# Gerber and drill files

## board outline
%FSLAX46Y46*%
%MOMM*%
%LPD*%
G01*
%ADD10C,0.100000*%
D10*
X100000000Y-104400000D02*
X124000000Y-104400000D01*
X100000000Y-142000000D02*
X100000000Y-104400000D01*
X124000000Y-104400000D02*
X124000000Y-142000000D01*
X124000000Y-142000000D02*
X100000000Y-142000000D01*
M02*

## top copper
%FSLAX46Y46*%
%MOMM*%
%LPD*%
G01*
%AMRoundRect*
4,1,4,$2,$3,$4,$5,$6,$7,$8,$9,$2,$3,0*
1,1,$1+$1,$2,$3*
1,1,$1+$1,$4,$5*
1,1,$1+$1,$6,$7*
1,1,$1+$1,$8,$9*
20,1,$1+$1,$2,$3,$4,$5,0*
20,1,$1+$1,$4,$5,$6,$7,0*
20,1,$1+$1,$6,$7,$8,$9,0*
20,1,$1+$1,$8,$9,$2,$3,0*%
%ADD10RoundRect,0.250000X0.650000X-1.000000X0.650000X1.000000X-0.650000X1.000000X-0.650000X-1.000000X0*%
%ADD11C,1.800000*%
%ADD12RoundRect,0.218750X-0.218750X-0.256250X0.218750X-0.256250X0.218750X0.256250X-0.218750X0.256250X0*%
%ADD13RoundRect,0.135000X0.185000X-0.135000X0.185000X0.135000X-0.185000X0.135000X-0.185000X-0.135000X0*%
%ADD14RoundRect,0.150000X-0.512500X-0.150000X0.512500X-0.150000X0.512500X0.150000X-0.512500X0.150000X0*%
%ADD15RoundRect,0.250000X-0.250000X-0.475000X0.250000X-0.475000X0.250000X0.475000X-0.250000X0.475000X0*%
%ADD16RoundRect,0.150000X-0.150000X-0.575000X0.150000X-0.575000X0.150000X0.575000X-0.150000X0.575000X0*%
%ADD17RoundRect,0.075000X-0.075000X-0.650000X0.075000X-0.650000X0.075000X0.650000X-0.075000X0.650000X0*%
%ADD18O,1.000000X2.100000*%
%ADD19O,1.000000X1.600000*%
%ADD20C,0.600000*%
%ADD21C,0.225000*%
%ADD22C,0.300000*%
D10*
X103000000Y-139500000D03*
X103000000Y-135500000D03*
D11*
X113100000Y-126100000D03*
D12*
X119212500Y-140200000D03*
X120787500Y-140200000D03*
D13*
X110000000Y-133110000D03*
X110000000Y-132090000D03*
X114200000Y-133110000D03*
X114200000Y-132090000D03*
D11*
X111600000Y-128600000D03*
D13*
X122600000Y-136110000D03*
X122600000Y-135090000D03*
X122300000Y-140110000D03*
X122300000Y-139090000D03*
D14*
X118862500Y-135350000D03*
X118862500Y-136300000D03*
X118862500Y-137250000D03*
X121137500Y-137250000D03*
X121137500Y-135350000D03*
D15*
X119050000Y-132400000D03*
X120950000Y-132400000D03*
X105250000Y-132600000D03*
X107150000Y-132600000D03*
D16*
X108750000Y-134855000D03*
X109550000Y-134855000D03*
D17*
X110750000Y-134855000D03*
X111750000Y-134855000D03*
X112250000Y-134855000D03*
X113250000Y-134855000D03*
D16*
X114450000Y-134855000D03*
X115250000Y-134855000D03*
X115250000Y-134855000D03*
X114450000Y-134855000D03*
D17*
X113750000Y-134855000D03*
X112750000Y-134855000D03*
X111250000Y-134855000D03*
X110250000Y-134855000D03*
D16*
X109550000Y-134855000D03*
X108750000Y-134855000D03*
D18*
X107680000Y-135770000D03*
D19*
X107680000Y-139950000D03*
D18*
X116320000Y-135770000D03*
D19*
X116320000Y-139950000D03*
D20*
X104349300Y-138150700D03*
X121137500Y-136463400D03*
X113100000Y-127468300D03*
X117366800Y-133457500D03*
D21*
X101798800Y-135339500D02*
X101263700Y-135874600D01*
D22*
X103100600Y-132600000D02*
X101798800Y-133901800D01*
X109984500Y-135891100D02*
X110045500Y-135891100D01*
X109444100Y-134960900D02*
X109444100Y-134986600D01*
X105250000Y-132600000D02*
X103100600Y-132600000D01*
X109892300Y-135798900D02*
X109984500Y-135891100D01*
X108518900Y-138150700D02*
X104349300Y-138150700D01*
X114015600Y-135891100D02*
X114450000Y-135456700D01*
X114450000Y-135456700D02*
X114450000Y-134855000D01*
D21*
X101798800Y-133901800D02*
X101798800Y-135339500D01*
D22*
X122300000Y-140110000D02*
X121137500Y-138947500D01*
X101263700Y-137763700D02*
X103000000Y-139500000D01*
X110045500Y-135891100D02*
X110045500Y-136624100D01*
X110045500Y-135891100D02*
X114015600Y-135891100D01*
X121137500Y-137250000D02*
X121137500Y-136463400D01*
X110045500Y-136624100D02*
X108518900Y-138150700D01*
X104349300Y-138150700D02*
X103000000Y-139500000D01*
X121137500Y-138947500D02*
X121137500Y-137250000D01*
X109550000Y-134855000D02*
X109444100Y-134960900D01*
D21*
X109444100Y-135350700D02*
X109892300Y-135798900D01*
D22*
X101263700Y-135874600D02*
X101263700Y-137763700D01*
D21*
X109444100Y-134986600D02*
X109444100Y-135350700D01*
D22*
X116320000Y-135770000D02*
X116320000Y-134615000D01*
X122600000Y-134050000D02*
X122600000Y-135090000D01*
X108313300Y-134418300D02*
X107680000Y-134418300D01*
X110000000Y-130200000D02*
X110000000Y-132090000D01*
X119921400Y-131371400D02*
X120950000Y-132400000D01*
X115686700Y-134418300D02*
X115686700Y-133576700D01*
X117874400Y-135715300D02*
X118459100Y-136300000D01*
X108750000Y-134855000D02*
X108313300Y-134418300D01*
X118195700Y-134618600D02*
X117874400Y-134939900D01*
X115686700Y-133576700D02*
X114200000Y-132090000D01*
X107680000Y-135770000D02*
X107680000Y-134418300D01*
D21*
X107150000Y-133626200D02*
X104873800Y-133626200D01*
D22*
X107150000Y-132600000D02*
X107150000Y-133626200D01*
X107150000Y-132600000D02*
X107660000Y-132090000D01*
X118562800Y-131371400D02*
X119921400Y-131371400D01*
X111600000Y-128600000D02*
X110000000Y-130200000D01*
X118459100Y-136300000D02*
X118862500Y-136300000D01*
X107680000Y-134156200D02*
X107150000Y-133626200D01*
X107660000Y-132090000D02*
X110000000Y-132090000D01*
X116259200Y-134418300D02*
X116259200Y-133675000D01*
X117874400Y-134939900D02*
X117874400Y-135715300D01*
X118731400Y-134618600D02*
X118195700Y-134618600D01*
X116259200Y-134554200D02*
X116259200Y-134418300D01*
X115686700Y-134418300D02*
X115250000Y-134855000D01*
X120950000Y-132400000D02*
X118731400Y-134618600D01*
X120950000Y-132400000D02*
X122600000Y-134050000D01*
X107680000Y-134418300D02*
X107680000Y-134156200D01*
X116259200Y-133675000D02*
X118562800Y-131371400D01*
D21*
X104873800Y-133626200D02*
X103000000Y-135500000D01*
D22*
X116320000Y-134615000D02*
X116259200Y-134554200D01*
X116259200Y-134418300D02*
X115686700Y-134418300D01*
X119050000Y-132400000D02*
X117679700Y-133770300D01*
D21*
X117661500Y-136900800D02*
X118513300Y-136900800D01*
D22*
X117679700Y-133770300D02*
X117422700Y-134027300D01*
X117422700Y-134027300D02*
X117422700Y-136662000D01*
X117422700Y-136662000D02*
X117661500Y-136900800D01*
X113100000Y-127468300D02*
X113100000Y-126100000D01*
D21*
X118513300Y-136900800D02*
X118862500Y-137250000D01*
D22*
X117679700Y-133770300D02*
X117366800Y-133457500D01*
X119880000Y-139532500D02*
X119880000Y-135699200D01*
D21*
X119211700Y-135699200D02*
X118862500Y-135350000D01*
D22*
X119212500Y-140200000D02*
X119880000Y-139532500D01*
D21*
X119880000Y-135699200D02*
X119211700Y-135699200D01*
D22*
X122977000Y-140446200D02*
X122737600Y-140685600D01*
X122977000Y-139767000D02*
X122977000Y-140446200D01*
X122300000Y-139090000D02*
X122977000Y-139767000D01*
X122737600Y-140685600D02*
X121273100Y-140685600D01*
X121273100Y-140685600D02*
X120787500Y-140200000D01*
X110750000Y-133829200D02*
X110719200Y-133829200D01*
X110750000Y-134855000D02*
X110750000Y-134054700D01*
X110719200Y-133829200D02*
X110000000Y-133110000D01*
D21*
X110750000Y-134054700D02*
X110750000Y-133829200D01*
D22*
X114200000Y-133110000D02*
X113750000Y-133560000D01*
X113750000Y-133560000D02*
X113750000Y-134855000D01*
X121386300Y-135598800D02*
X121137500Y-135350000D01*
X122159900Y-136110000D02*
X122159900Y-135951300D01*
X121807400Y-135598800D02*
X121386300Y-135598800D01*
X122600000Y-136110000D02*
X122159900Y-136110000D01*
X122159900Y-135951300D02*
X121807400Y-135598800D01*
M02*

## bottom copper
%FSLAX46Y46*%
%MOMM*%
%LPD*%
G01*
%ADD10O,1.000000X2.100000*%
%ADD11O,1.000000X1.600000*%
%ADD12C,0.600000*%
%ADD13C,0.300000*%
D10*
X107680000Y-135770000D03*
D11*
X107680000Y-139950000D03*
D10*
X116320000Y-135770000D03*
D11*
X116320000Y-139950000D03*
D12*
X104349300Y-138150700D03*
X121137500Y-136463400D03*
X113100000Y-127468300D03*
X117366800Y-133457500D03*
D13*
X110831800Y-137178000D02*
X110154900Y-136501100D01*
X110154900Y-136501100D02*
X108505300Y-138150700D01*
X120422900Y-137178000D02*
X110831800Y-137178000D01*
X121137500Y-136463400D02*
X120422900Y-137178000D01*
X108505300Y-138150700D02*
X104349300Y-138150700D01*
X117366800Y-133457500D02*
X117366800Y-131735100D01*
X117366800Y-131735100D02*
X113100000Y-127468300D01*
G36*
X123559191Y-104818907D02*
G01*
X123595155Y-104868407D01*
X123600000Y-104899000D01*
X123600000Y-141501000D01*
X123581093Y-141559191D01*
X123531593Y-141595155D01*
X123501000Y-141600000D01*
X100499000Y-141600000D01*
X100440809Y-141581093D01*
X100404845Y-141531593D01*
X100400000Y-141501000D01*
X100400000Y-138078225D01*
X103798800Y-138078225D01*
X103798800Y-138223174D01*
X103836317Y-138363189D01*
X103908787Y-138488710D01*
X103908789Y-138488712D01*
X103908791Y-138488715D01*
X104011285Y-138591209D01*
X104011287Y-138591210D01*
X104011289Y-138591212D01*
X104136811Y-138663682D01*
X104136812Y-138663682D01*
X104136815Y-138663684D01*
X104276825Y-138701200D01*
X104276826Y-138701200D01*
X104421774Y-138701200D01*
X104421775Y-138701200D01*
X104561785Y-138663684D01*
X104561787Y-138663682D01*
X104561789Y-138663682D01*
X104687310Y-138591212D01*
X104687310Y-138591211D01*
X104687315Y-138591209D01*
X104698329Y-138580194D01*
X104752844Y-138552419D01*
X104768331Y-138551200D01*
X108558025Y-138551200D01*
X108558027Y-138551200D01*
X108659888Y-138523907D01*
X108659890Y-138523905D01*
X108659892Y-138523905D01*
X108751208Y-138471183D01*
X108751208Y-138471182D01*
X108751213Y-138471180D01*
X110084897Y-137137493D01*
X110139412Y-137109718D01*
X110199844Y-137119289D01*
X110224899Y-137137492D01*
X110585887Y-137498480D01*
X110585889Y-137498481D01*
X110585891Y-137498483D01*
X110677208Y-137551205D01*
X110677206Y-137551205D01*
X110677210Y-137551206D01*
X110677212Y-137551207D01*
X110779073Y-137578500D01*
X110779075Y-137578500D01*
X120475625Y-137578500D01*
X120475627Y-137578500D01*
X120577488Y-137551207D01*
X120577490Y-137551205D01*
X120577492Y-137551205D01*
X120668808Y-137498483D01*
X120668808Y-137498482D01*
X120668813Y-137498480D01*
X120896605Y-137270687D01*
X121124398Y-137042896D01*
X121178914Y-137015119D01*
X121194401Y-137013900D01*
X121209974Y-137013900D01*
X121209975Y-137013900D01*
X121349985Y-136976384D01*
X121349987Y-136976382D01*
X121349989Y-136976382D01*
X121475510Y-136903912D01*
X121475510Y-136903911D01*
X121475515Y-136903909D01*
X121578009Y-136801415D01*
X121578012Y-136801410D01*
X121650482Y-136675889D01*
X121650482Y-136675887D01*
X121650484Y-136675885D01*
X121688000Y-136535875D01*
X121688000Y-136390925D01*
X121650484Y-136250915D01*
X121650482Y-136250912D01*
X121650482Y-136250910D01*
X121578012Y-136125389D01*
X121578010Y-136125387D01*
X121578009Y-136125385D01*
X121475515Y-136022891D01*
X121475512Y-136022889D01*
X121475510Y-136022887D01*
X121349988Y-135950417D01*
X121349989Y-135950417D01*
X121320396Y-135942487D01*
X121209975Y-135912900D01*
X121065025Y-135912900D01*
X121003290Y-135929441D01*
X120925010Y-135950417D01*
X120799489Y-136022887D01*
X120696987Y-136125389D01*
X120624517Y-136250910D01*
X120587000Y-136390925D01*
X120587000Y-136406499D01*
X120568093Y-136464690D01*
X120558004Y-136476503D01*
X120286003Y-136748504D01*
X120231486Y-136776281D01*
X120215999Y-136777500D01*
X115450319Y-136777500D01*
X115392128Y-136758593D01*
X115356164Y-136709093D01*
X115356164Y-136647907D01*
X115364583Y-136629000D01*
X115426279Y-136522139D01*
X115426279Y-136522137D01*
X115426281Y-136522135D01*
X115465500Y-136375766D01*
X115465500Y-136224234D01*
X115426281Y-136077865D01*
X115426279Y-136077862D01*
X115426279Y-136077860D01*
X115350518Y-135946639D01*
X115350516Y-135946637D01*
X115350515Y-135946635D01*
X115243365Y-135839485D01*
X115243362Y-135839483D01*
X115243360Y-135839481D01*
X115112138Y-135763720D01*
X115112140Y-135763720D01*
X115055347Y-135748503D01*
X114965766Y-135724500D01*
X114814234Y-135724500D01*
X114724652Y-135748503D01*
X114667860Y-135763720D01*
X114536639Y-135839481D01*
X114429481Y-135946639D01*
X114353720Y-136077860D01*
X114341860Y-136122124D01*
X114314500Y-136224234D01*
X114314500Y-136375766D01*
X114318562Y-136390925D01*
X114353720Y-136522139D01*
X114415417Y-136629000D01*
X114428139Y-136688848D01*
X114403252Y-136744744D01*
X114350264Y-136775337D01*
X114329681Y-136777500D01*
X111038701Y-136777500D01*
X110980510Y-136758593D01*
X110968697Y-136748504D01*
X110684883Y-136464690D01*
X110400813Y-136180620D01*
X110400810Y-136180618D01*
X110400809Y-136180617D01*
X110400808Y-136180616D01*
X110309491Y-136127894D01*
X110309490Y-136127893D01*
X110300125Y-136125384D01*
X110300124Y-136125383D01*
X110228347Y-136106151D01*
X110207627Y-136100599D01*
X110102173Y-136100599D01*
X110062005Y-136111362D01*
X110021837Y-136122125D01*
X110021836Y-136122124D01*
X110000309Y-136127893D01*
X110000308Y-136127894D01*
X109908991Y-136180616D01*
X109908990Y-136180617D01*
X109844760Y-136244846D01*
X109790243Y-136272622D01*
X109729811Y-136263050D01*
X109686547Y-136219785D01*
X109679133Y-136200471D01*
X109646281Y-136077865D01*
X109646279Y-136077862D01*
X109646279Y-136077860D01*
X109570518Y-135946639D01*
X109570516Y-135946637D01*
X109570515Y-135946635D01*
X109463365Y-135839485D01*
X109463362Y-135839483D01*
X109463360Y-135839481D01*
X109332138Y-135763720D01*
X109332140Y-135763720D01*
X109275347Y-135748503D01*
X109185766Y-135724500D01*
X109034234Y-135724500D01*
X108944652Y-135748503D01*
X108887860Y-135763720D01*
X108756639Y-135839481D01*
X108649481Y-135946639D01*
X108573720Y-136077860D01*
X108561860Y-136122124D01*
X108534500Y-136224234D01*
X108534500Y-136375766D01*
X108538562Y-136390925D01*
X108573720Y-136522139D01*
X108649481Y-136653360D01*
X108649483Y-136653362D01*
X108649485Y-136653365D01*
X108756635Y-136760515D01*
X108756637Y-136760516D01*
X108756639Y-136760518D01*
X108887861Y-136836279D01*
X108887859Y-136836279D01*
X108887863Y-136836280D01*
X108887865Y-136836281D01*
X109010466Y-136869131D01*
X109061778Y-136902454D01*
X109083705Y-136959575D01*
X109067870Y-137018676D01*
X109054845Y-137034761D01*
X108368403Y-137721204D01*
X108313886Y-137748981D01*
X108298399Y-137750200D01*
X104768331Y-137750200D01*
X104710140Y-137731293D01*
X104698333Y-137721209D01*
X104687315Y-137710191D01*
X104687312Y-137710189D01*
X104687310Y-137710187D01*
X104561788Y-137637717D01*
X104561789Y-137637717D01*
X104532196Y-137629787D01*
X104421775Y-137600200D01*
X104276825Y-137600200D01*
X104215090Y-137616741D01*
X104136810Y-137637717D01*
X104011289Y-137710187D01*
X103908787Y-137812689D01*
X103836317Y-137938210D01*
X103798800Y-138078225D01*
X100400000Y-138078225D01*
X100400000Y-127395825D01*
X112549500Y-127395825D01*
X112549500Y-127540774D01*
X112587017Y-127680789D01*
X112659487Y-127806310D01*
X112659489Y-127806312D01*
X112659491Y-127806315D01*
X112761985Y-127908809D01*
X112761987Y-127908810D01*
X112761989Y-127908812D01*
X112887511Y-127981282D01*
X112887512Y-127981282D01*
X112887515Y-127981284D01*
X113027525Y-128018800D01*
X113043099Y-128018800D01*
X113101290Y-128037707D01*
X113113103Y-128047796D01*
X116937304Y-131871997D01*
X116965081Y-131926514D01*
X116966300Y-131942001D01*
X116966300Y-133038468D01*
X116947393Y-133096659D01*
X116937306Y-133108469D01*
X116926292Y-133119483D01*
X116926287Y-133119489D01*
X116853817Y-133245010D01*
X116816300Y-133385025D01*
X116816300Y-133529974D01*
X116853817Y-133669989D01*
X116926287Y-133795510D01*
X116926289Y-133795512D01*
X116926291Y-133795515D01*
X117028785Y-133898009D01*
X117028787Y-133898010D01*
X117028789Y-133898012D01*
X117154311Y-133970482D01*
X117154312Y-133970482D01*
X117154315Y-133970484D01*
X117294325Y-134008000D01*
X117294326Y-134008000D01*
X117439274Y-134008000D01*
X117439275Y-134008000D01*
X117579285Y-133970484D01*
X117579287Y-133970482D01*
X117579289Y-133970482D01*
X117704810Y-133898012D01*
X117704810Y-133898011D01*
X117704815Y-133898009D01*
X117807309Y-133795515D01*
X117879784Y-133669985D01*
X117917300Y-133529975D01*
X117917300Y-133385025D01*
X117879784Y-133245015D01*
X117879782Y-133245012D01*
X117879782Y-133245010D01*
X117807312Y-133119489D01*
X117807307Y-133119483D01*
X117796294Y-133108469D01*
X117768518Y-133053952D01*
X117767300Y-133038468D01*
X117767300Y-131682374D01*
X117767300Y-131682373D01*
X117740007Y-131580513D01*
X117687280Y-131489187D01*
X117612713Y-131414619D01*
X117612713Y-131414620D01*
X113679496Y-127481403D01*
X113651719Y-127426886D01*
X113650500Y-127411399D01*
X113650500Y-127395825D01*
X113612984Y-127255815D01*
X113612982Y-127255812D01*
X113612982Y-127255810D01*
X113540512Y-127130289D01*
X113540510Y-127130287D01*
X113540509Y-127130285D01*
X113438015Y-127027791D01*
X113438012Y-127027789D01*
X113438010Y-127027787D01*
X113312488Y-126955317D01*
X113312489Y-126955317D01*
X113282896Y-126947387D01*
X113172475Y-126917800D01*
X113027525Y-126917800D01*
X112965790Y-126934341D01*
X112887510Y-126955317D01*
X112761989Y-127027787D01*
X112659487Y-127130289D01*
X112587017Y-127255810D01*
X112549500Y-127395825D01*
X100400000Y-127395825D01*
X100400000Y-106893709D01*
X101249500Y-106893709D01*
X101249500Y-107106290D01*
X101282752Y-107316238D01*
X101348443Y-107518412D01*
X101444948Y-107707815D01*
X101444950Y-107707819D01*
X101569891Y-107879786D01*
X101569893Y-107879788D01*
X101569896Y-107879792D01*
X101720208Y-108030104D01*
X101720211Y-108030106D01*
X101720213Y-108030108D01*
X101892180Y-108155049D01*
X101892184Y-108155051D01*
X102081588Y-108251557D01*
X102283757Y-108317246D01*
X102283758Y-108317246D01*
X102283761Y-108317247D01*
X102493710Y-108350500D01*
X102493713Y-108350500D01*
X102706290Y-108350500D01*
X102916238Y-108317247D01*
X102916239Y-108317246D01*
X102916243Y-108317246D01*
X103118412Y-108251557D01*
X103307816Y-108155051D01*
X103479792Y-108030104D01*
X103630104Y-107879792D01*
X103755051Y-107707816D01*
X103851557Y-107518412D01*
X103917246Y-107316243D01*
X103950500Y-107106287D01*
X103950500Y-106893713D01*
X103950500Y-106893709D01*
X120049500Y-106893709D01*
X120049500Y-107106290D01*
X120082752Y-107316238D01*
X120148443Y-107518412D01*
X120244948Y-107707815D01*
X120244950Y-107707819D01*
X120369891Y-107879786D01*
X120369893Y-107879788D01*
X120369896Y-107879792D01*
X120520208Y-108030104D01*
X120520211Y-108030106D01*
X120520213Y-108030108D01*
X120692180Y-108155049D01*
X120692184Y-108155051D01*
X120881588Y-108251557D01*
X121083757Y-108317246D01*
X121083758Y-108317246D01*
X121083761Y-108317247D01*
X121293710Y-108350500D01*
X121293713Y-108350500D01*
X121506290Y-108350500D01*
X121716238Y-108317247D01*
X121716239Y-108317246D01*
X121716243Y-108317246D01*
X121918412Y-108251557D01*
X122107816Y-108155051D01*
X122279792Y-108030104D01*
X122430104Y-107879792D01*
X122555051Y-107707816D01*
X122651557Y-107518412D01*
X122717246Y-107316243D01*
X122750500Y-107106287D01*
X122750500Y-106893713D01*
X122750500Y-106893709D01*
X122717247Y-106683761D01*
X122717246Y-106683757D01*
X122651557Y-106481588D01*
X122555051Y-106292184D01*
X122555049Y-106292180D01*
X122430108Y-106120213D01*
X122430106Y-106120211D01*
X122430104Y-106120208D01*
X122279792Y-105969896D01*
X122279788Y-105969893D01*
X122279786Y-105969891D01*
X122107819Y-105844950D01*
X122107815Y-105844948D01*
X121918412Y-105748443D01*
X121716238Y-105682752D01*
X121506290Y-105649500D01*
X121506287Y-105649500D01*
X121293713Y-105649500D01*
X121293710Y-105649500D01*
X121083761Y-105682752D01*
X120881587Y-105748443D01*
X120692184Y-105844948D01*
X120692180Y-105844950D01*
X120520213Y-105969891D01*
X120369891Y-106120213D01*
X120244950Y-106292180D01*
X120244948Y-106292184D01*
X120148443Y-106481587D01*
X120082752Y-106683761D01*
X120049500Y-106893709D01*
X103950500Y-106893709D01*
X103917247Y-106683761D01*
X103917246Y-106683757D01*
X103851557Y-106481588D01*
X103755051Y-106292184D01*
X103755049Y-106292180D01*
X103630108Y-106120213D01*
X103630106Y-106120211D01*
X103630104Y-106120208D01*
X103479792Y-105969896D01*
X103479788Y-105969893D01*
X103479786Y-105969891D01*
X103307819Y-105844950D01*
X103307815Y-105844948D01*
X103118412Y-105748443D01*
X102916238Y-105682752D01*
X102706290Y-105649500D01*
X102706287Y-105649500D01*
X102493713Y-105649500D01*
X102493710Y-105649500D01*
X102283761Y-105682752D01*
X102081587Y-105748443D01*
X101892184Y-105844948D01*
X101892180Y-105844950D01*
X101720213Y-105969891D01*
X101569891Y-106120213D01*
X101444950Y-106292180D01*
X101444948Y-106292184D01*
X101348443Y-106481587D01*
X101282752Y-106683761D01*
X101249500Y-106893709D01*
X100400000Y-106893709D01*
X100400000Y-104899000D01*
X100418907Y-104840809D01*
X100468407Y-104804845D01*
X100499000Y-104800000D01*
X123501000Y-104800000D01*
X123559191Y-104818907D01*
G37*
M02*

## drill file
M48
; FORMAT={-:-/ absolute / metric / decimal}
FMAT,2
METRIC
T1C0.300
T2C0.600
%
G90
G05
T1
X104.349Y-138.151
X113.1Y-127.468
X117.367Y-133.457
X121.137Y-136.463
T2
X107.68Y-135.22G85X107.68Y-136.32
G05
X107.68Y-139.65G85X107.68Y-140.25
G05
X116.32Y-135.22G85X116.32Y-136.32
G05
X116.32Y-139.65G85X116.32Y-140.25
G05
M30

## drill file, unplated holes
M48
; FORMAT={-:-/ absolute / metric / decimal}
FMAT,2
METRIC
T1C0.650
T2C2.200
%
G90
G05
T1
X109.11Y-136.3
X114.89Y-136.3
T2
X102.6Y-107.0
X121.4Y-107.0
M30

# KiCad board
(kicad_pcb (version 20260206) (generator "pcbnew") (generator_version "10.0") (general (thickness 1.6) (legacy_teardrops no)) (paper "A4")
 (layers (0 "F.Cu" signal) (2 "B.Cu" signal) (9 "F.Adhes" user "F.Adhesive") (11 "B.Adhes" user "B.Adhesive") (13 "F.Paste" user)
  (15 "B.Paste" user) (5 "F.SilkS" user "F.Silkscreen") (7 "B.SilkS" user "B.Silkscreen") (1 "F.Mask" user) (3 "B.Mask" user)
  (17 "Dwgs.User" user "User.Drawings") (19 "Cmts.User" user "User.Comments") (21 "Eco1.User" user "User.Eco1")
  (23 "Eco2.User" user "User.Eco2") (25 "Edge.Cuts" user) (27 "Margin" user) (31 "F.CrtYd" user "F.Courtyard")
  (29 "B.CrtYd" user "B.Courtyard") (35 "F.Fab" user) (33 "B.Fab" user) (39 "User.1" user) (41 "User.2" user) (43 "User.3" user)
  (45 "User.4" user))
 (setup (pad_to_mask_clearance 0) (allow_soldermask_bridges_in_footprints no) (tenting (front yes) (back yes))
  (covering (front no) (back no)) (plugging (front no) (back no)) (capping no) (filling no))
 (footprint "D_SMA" (layer "F.Cu") (at 103 137.5 90)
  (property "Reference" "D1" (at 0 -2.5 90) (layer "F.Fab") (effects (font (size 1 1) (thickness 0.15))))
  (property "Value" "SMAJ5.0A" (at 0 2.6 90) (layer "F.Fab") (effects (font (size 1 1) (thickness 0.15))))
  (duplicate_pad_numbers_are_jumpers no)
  (pad "1" smd roundrect (at -2 0 90) (size 2.5 1.8) (layers "F.Cu" "F.Mask" "F.Paste") (roundrect_rratio 0.1388888889) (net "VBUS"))
  (pad "2" smd roundrect (at 2 0 90) (size 2.5 1.8) (layers "F.Cu" "F.Mask" "F.Paste") (roundrect_rratio 0.1388888889) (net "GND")))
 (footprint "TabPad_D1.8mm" (layer "F.Cu") (at 113.1 126.1)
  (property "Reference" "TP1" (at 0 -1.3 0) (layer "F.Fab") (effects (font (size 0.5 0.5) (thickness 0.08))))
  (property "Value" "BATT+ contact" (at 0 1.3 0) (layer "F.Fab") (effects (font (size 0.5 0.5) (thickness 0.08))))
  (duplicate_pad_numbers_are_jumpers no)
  (pad "1" smd circle (at 0 0) (size 1.8 1.8) (layers "F.Cu" "F.Mask") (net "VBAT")))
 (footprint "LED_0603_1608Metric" (layer "F.Cu") (at 120 140.2)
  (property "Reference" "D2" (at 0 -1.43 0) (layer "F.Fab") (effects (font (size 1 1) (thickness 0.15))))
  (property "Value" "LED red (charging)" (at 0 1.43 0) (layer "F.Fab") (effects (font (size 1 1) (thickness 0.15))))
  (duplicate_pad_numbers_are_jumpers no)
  (pad "1" smd roundrect (at -0.7875 0) (size 0.875 0.95) (layers "F.Cu" "F.Mask" "F.Paste") (roundrect_rratio 0.25) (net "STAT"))
  (pad "2" smd roundrect (at 0.7875 0) (size 0.875 0.95) (layers "F.Cu" "F.Mask" "F.Paste") (roundrect_rratio 0.25) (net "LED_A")))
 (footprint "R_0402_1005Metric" (layer "F.Cu") (at 110 132.6 90)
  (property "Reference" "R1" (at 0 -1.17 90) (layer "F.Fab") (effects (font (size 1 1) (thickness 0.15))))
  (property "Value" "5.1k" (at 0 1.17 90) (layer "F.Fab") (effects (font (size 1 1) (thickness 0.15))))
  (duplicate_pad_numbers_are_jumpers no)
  (pad "1" smd roundrect (at -0.51 0 90) (size 0.54 0.64) (layers "F.Cu" "F.Mask" "F.Paste") (roundrect_rratio 0.25) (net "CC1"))
  (pad "2" smd roundrect (at 0.51 0 90) (size 0.54 0.64) (layers "F.Cu" "F.Mask" "F.Paste") (roundrect_rratio 0.25) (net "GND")))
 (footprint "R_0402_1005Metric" (layer "F.Cu") (at 114.2 132.6 90)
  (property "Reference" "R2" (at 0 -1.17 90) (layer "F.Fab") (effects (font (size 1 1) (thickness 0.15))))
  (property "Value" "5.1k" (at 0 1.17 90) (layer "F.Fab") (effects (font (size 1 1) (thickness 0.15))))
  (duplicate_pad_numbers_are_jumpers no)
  (pad "1" smd roundrect (at -0.51 0 90) (size 0.54 0.64) (layers "F.Cu" "F.Mask" "F.Paste") (roundrect_rratio 0.25) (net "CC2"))
  (pad "2" smd roundrect (at 0.51 0 90) (size 0.54 0.64) (layers "F.Cu" "F.Mask" "F.Paste") (roundrect_rratio 0.25) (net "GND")))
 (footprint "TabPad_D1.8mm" (layer "F.Cu") (at 111.6 128.6)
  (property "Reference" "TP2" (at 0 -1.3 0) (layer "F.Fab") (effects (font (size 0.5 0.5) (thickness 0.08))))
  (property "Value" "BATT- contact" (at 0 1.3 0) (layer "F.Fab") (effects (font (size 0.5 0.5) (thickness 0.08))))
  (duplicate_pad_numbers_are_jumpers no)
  (pad "1" smd circle (at 0 0) (size 1.8 1.8) (layers "F.Cu" "F.Mask") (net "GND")))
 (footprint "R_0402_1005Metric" (layer "F.Cu") (at 122.6 135.6 90)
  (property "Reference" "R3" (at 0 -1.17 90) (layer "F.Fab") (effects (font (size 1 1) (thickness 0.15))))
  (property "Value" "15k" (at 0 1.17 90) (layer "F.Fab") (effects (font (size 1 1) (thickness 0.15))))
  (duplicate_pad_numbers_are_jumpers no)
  (pad "1" smd roundrect (at -0.51 0 90) (size 0.54 0.64) (layers "F.Cu" "F.Mask" "F.Paste") (roundrect_rratio 0.25) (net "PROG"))
  (pad "2" smd roundrect (at 0.51 0 90) (size 0.54 0.64) (layers "F.Cu" "F.Mask" "F.Paste") (roundrect_rratio 0.25) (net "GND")))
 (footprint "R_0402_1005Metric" (layer "F.Cu") (at 122.3 139.6 90)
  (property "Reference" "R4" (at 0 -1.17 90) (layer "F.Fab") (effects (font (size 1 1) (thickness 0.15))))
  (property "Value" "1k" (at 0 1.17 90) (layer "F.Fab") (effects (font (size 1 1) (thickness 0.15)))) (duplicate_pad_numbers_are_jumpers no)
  (pad "1" smd roundrect (at -0.51 0 90) (size 0.54 0.64) (layers "F.Cu" "F.Mask" "F.Paste") (roundrect_rratio 0.25) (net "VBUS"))
  (pad "2" smd roundrect (at 0.51 0 90) (size 0.54 0.64) (layers "F.Cu" "F.Mask" "F.Paste") (roundrect_rratio 0.25) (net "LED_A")))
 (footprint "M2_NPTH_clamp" (layer "F.Cu") (at 121.4 107)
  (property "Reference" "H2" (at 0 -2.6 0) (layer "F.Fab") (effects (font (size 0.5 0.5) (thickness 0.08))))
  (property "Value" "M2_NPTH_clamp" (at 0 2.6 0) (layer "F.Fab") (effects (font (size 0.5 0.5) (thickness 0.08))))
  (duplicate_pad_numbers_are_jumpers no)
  (pad "" np_thru_hole circle (at 0 0) (size 2.2 2.2) (drill 2.2) (layers "*.Cu" "*.Mask")))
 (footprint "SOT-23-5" (layer "F.Cu") (at 120 136.3)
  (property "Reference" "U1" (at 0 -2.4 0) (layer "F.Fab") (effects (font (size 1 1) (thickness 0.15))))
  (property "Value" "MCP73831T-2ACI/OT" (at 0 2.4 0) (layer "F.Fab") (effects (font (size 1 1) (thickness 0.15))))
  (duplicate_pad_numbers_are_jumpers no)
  (pad "1" smd roundrect (at -1.1375 -0.95) (size 1.325 0.6) (layers "F.Cu" "F.Mask" "F.Paste") (roundrect_rratio 0.25) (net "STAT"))
  (pad "2" smd roundrect (at -1.1375 0) (size 1.325 0.6) (layers "F.Cu" "F.Mask" "F.Paste") (roundrect_rratio 0.25) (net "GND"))
  (pad "3" smd roundrect (at -1.1375 0.95) (size 1.325 0.6) (layers "F.Cu" "F.Mask" "F.Paste") (roundrect_rratio 0.25) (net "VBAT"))
  (pad "4" smd roundrect (at 1.1375 0.95) (size 1.325 0.6) (layers "F.Cu" "F.Mask" "F.Paste") (roundrect_rratio 0.25) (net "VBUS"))
  (pad "5" smd roundrect (at 1.1375 -0.95) (size 1.325 0.6) (layers "F.Cu" "F.Mask" "F.Paste") (roundrect_rratio 0.25) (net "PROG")))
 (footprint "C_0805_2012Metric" (layer "F.Cu") (at 120 132.4)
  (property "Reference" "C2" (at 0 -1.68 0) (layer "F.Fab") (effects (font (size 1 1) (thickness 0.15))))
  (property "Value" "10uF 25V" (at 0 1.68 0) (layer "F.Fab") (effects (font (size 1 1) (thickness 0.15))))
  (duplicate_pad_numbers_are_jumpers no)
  (pad "1" smd roundrect (at -0.95 0) (size 1 1.45) (layers "F.Cu" "F.Mask" "F.Paste") (roundrect_rratio 0.25) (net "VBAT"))
  (pad "2" smd roundrect (at 0.95 0) (size 1 1.45) (layers "F.Cu" "F.Mask" "F.Paste") (roundrect_rratio 0.25) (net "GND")))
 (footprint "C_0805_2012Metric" (layer "F.Cu") (at 106.2 132.6)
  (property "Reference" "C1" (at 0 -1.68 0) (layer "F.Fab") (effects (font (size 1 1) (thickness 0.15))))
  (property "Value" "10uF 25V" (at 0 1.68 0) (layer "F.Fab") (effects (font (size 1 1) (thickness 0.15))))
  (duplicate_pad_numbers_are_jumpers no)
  (pad "1" smd roundrect (at -0.95 0) (size 1 1.45) (layers "F.Cu" "F.Mask" "F.Paste") (roundrect_rratio 0.25) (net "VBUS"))
  (pad "2" smd roundrect (at 0.95 0) (size 1 1.45) (layers "F.Cu" "F.Mask" "F.Paste") (roundrect_rratio 0.25) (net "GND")))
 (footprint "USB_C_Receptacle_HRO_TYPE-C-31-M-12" (layer "F.Cu") (at 112 138.9)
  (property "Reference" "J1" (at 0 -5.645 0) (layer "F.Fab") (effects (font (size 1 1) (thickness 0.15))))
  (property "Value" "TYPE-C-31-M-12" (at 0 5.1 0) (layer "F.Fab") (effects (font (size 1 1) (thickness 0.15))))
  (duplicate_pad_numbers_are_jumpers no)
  (pad "" np_thru_hole circle (at -2.89 -2.6) (size 0.65 0.65) (drill 0.65) (layers "*.Cu" "*.Mask"))
  (pad "" np_thru_hole circle (at 2.89 -2.6) (size 0.65 0.65) (drill 0.65) (layers "*.Cu" "*.Mask"))
  (pad "A1" smd roundrect (at -3.25 -4.045) (size 0.6 1.45) (layers "F.Cu" "F.Mask" "F.Paste") (roundrect_rratio 0.25) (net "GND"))
  (pad "A4" smd roundrect (at -2.45 -4.045) (size 0.6 1.45) (layers "F.Cu" "F.Mask" "F.Paste") (roundrect_rratio 0.25) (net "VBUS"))
  (pad "A5" smd roundrect (at -1.25 -4.045) (size 0.3 1.45) (layers "F.Cu" "F.Mask" "F.Paste") (roundrect_rratio 0.25) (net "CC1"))
  (pad "A6" smd roundrect (at -0.25 -4.045) (size 0.3 1.45) (layers "F.Cu" "F.Mask" "F.Paste") (roundrect_rratio 0.25))
  (pad "A7" smd roundrect (at 0.25 -4.045) (size 0.3 1.45) (layers "F.Cu" "F.Mask" "F.Paste") (roundrect_rratio 0.25))
  (pad "A8" smd roundrect (at 1.25 -4.045) (size 0.3 1.45) (layers "F.Cu" "F.Mask" "F.Paste") (roundrect_rratio 0.25))
  (pad "A9" smd roundrect (at 2.45 -4.045) (size 0.6 1.45) (layers "F.Cu" "F.Mask" "F.Paste") (roundrect_rratio 0.25) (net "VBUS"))
  (pad "A12" smd roundrect (at 3.25 -4.045) (size 0.6 1.45) (layers "F.Cu" "F.Mask" "F.Paste") (roundrect_rratio 0.25) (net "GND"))
  (pad "B1" smd roundrect (at 3.25 -4.045) (size 0.6 1.45) (layers "F.Cu" "F.Mask" "F.Paste") (roundrect_rratio 0.25) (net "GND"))
  (pad "B4" smd roundrect (at 2.45 -4.045) (size 0.6 1.45) (layers "F.Cu" "F.Mask" "F.Paste") (roundrect_rratio 0.25) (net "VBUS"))
  (pad "B5" smd roundrect (at 1.75 -4.045) (size 0.3 1.45) (layers "F.Cu" "F.Mask" "F.Paste") (roundrect_rratio 0.25) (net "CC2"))
  (pad "B6" smd roundrect (at 0.75 -4.045) (size 0.3 1.45) (layers "F.Cu" "F.Mask" "F.Paste") (roundrect_rratio 0.25))
  (pad "B7" smd roundrect (at -0.75 -4.045) (size 0.3 1.45) (layers "F.Cu" "F.Mask" "F.Paste") (roundrect_rratio 0.25))
  (pad "B8" smd roundrect (at -1.75 -4.045) (size 0.3 1.45) (layers "F.Cu" "F.Mask" "F.Paste") (roundrect_rratio 0.25))
  (pad "B9" smd roundrect (at -2.45 -4.045) (size 0.6 1.45) (layers "F.Cu" "F.Mask" "F.Paste") (roundrect_rratio 0.25) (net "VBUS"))
  (pad "B12" smd roundrect (at -3.25 -4.045) (size 0.6 1.45) (layers "F.Cu" "F.Mask" "F.Paste") (roundrect_rratio 0.25) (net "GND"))
  (pad "SH" thru_hole oval (at -4.32 -3.13) (size 1 2.1) (drill oval 0.6 1.7) (layers "*.Cu" "*.Mask") (remove_unused_layers no) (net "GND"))
  (pad "SH" thru_hole oval (at -4.32 1.05) (size 1 1.6) (drill oval 0.6 1.2) (layers "*.Cu" "*.Mask") (remove_unused_layers no) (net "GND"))
  (pad "SH" thru_hole oval (at 4.32 -3.13) (size 1 2.1) (drill oval 0.6 1.7) (layers "*.Cu" "*.Mask") (remove_unused_layers no) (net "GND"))
  (pad "SH" thru_hole oval (at 4.32 1.05) (size 1 1.6) (drill oval 0.6 1.2) (layers "*.Cu" "*.Mask") (remove_unused_layers no) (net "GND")))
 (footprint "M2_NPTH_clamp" (layer "F.Cu") (at 102.6 107)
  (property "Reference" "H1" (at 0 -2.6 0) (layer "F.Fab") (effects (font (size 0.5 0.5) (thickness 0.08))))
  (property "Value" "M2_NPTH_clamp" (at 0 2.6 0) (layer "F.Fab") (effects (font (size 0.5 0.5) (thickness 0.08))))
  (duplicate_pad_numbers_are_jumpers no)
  (pad "" np_thru_hole circle (at 0 0) (size 2.2 2.2) (drill 2.2) (layers "*.Cu" "*.Mask")))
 (gr_line (start 100 104.4) (end 124 104.4) (stroke (width 0.1) (type default)) (layer "Edge.Cuts"))
 (gr_line (start 100 142) (end 100 104.4) (stroke (width 0.1) (type default)) (layer "Edge.Cuts"))
 (gr_line (start 124 104.4) (end 124 142) (stroke (width 0.1) (type default)) (layer "Edge.Cuts"))
 (gr_line (start 124 142) (end 100 142) (stroke (width 0.1) (type default)) (layer "Edge.Cuts"))
 (segment (start 101.7988 135.3395) (end 101.2637 135.8746) (width 0.225) (layer "F.Cu") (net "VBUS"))
 (segment (start 103.1006 132.6) (end 101.7988 133.9018) (width 0.3) (layer "F.Cu") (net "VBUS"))
 (segment (start 109.9845 135.8911) (end 110.0455 135.8911) (width 0.3) (layer "F.Cu") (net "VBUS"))
 (segment (start 109.4441 134.9609) (end 109.4441 134.9866) (width 0.3) (layer "F.Cu") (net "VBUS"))
 (segment (start 105.25 132.6) (end 103.1006 132.6) (width 0.3) (layer "F.Cu") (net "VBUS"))
 (segment (start 109.8923 135.7989) (end 109.9845 135.8911) (width 0.3) (layer "F.Cu") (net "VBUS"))
 (segment (start 108.5189 138.1507) (end 104.3493 138.1507) (width 0.3) (layer "F.Cu") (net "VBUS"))
 (segment (start 114.0156 135.8911) (end 114.45 135.4567) (width 0.3) (layer "F.Cu") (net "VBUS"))
 (segment (start 114.45 135.4567) (end 114.45 134.855) (width 0.3) (layer "F.Cu") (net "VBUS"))
 (segment (start 101.7988 133.9018) (end 101.7988 135.3395) (width 0.225) (layer "F.Cu") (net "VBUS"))
 (segment (start 122.3 140.11) (end 121.1375 138.9475) (width 0.3) (layer "F.Cu") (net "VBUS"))
 (segment (start 101.2637 137.7637) (end 103 139.5) (width 0.3) (layer "F.Cu") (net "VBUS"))
 (segment (start 110.0455 135.8911) (end 110.0455 136.6241) (width 0.3) (layer "F.Cu") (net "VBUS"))
 (segment (start 110.0455 135.8911) (end 114.0156 135.8911) (width 0.3) (layer "F.Cu") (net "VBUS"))
 (segment (start 121.1375 137.25) (end 121.1375 136.4634) (width 0.3) (layer "F.Cu") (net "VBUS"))
 (segment (start 110.0455 136.6241) (end 108.5189 138.1507) (width 0.3) (layer "F.Cu") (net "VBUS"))
 (segment (start 104.3493 138.1507) (end 103 139.5) (width 0.3) (layer "F.Cu") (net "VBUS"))
 (segment (start 121.1375 138.9475) (end 121.1375 137.25) (width 0.3) (layer "F.Cu") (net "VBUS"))
 (segment (start 109.55 134.855) (end 109.4441 134.9609) (width 0.3) (layer "F.Cu") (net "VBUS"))
 (segment (start 109.4441 135.3507) (end 109.8923 135.7989) (width 0.225) (layer "F.Cu") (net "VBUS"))
 (segment (start 101.2637 135.8746) (end 101.2637 137.7637) (width 0.3) (layer "F.Cu") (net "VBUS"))
 (segment (start 109.4441 134.9866) (end 109.4441 135.3507) (width 0.225) (layer "F.Cu") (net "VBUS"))
 (via (at 104.3493 138.1507) (size 0.6) (drill 0.3) (layers "F.Cu" "B.Cu") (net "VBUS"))
 (via (at 121.1375 136.4634) (size 0.6) (drill 0.3) (layers "F.Cu" "B.Cu") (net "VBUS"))
 (segment (start 110.8318 137.178) (end 110.1549 136.5011) (width 0.3) (layer "B.Cu") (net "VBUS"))
 (segment (start 110.1549 136.5011) (end 108.5053 138.1507) (width 0.3) (layer "B.Cu") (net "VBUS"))
 (segment (start 120.4229 137.178) (end 110.8318 137.178) (width 0.3) (layer "B.Cu") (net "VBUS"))
 (segment (start 121.1375 136.4634) (end 120.4229 137.178) (width 0.3) (layer "B.Cu") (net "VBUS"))
 (segment (start 108.5053 138.1507) (end 104.3493 138.1507) (width 0.3) (layer "B.Cu") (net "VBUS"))
 (segment (start 116.32 135.77) (end 116.32 134.615) (width 0.3) (layer "F.Cu") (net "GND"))
 (segment (start 122.6 134.05) (end 122.6 135.09) (width 0.3) (layer "F.Cu") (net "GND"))
 (segment (start 108.3133 134.4183) (end 107.68 134.4183) (width 0.3) (layer "F.Cu") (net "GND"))
 (segment (start 110 130.2) (end 110 132.09) (width 0.3) (layer "F.Cu") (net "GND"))
 (segment (start 119.9214 131.3714) (end 120.95 132.4) (width 0.3) (layer "F.Cu") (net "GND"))
 (segment (start 115.6867 134.4183) (end 115.6867 133.5767) (width 0.3) (layer "F.Cu") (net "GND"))
 (segment (start 117.8744 135.7153) (end 118.4591 136.3) (width 0.3) (layer "F.Cu") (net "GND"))
 (segment (start 108.75 134.855) (end 108.3133 134.4183) (width 0.3) (layer "F.Cu") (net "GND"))
 (segment (start 118.1957 134.6186) (end 117.8744 134.9399) (width 0.3) (layer "F.Cu") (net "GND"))
 (segment (start 115.6867 133.5767) (end 114.2 132.09) (width 0.3) (layer "F.Cu") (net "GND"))
 (segment (start 107.68 135.77) (end 107.68 134.4183) (width 0.3) (layer "F.Cu") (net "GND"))
 (segment (start 107.15 133.6262) (end 104.8738 133.6262) (width 0.225) (layer "F.Cu") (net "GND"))
 (segment (start 107.15 132.6) (end 107.15 133.6262) (width 0.3) (layer "F.Cu") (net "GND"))
 (segment (start 107.15 132.6) (end 107.66 132.09) (width 0.3) (layer "F.Cu") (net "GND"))
 (segment (start 118.5628 131.3714) (end 119.9214 131.3714) (width 0.3) (layer "F.Cu") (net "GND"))
 (segment (start 111.6 128.6) (end 110 130.2) (width 0.3) (layer "F.Cu") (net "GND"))
 (segment (start 118.4591 136.3) (end 118.8625 136.3) (width 0.3) (layer "F.Cu") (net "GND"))
 (segment (start 107.68 134.1562) (end 107.15 133.6262) (width 0.3) (layer "F.Cu") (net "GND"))
 (segment (start 107.66 132.09) (end 110 132.09) (width 0.3) (layer "F.Cu") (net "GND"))
 (segment (start 116.2592 134.4183) (end 116.2592 133.675) (width 0.3) (layer "F.Cu") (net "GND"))
 (segment (start 117.8744 134.9399) (end 117.8744 135.7153) (width 0.3) (layer "F.Cu") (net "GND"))
 (segment (start 118.7314 134.6186) (end 118.1957 134.6186) (width 0.3) (layer "F.Cu") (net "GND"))
 (segment (start 116.2592 134.5542) (end 116.2592 134.4183) (width 0.3) (layer "F.Cu") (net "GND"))
 (segment (start 115.6867 134.4183) (end 115.25 134.855) (width 0.3) (layer "F.Cu") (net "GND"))
 (segment (start 120.95 132.4) (end 118.7314 134.6186) (width 0.3) (layer "F.Cu") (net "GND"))
 (segment (start 120.95 132.4) (end 122.6 134.05) (width 0.3) (layer "F.Cu") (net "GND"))
 (segment (start 107.68 134.4183) (end 107.68 134.1562) (width 0.3) (layer "F.Cu") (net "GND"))
 (segment (start 116.2592 133.675) (end 118.5628 131.3714) (width 0.3) (layer "F.Cu") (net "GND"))
 (segment (start 104.8738 133.6262) (end 103 135.5) (width 0.225) (layer "F.Cu") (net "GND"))
 (segment (start 116.32 134.615) (end 116.2592 134.5542) (width 0.3) (layer "F.Cu") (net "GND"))
 (segment (start 116.2592 134.4183) (end 115.6867 134.4183) (width 0.3) (layer "F.Cu") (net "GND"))
 (segment (start 119.05 132.4) (end 117.6797 133.7703) (width 0.3) (layer "F.Cu") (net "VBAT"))
 (segment (start 117.6615 136.9008) (end 118.5133 136.9008) (width 0.225) (layer "F.Cu") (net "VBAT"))
 (segment (start 117.6797 133.7703) (end 117.4227 134.0273) (width 0.3) (layer "F.Cu") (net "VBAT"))
 (segment (start 117.4227 134.0273) (end 117.4227 136.662) (width 0.3) (layer "F.Cu") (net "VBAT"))
 (segment (start 117.4227 136.662) (end 117.6615 136.9008) (width 0.3) (layer "F.Cu") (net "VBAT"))
 (segment (start 113.1 127.4683) (end 113.1 126.1) (width 0.3) (layer "F.Cu") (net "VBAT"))
 (segment (start 118.5133 136.9008) (end 118.8625 137.25) (width 0.225) (layer "F.Cu") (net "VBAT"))
 (segment (start 117.6797 133.7703) (end 117.3668 133.4575) (width 0.3) (layer "F.Cu") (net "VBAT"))
 (via (at 113.1 127.4683) (size 0.6) (drill 0.3) (layers "F.Cu" "B.Cu") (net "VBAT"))
 (via (at 117.3668 133.4575) (size 0.6) (drill 0.3) (layers "F.Cu" "B.Cu") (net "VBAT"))
 (segment (start 117.3668 133.4575) (end 117.3668 131.7351) (width 0.3) (layer "B.Cu") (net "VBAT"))
 (segment (start 117.3668 131.7351) (end 113.1 127.4683) (width 0.3) (layer "B.Cu") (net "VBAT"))
 (segment (start 119.88 139.5325) (end 119.88 135.6992) (width 0.3) (layer "F.Cu") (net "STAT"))
 (segment (start 119.2117 135.6992) (end 118.8625 135.35) (width 0.225) (layer "F.Cu") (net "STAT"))
 (segment (start 119.2125 140.2) (end 119.88 139.5325) (width 0.3) (layer "F.Cu") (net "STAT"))
 (segment (start 119.88 135.6992) (end 119.2117 135.6992) (width 0.225) (layer "F.Cu") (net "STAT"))
 (segment (start 122.977 140.4462) (end 122.7376 140.6856) (width 0.3) (layer "F.Cu") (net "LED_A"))
 (segment (start 122.977 139.767) (end 122.977 140.4462) (width 0.3) (layer "F.Cu") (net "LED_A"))
 (segment (start 122.3 139.09) (end 122.977 139.767) (width 0.3) (layer "F.Cu") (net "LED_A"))
 (segment (start 122.7376 140.6856) (end 121.2731 140.6856) (width 0.3) (layer "F.Cu") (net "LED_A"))
 (segment (start 121.2731 140.6856) (end 120.7875 140.2) (width 0.3) (layer "F.Cu") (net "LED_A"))
 (segment (start 110.75 133.8292) (end 110.7192 133.8292) (width 0.3) (layer "F.Cu") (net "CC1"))
 (segment (start 110.75 134.855) (end 110.75 134.0547) (width 0.3) (layer "F.Cu") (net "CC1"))
 (segment (start 110.7192 133.8292) (end 110 133.11) (width 0.3) (layer "F.Cu") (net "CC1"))
 (segment (start 110.75 134.0547) (end 110.75 133.8292) (width 0.225) (layer "F.Cu") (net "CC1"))
 (segment (start 114.2 133.11) (end 113.75 133.56) (width 0.3) (layer "F.Cu") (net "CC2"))
 (segment (start 113.75 133.56) (end 113.75 134.855) (width 0.3) (layer "F.Cu") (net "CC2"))
 (segment (start 121.3863 135.5988) (end 121.1375 135.35) (width 0.3) (layer "F.Cu") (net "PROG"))
 (segment (start 122.1599 136.11) (end 122.1599 135.9513) (width 0.3) (layer "F.Cu") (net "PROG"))
 (segment (start 121.8074 135.5988) (end 121.3863 135.5988) (width 0.3) (layer "F.Cu") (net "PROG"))
 (segment (start 122.6 136.11) (end 122.1599 136.11) (width 0.3) (layer "F.Cu") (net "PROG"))
 (segment (start 122.1599 135.9513) (end 121.8074 135.5988) (width 0.3) (layer "F.Cu") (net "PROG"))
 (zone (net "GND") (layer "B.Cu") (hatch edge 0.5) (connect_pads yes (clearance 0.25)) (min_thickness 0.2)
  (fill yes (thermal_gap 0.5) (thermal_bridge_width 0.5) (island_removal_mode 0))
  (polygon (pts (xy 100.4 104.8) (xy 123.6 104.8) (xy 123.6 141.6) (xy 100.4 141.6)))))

